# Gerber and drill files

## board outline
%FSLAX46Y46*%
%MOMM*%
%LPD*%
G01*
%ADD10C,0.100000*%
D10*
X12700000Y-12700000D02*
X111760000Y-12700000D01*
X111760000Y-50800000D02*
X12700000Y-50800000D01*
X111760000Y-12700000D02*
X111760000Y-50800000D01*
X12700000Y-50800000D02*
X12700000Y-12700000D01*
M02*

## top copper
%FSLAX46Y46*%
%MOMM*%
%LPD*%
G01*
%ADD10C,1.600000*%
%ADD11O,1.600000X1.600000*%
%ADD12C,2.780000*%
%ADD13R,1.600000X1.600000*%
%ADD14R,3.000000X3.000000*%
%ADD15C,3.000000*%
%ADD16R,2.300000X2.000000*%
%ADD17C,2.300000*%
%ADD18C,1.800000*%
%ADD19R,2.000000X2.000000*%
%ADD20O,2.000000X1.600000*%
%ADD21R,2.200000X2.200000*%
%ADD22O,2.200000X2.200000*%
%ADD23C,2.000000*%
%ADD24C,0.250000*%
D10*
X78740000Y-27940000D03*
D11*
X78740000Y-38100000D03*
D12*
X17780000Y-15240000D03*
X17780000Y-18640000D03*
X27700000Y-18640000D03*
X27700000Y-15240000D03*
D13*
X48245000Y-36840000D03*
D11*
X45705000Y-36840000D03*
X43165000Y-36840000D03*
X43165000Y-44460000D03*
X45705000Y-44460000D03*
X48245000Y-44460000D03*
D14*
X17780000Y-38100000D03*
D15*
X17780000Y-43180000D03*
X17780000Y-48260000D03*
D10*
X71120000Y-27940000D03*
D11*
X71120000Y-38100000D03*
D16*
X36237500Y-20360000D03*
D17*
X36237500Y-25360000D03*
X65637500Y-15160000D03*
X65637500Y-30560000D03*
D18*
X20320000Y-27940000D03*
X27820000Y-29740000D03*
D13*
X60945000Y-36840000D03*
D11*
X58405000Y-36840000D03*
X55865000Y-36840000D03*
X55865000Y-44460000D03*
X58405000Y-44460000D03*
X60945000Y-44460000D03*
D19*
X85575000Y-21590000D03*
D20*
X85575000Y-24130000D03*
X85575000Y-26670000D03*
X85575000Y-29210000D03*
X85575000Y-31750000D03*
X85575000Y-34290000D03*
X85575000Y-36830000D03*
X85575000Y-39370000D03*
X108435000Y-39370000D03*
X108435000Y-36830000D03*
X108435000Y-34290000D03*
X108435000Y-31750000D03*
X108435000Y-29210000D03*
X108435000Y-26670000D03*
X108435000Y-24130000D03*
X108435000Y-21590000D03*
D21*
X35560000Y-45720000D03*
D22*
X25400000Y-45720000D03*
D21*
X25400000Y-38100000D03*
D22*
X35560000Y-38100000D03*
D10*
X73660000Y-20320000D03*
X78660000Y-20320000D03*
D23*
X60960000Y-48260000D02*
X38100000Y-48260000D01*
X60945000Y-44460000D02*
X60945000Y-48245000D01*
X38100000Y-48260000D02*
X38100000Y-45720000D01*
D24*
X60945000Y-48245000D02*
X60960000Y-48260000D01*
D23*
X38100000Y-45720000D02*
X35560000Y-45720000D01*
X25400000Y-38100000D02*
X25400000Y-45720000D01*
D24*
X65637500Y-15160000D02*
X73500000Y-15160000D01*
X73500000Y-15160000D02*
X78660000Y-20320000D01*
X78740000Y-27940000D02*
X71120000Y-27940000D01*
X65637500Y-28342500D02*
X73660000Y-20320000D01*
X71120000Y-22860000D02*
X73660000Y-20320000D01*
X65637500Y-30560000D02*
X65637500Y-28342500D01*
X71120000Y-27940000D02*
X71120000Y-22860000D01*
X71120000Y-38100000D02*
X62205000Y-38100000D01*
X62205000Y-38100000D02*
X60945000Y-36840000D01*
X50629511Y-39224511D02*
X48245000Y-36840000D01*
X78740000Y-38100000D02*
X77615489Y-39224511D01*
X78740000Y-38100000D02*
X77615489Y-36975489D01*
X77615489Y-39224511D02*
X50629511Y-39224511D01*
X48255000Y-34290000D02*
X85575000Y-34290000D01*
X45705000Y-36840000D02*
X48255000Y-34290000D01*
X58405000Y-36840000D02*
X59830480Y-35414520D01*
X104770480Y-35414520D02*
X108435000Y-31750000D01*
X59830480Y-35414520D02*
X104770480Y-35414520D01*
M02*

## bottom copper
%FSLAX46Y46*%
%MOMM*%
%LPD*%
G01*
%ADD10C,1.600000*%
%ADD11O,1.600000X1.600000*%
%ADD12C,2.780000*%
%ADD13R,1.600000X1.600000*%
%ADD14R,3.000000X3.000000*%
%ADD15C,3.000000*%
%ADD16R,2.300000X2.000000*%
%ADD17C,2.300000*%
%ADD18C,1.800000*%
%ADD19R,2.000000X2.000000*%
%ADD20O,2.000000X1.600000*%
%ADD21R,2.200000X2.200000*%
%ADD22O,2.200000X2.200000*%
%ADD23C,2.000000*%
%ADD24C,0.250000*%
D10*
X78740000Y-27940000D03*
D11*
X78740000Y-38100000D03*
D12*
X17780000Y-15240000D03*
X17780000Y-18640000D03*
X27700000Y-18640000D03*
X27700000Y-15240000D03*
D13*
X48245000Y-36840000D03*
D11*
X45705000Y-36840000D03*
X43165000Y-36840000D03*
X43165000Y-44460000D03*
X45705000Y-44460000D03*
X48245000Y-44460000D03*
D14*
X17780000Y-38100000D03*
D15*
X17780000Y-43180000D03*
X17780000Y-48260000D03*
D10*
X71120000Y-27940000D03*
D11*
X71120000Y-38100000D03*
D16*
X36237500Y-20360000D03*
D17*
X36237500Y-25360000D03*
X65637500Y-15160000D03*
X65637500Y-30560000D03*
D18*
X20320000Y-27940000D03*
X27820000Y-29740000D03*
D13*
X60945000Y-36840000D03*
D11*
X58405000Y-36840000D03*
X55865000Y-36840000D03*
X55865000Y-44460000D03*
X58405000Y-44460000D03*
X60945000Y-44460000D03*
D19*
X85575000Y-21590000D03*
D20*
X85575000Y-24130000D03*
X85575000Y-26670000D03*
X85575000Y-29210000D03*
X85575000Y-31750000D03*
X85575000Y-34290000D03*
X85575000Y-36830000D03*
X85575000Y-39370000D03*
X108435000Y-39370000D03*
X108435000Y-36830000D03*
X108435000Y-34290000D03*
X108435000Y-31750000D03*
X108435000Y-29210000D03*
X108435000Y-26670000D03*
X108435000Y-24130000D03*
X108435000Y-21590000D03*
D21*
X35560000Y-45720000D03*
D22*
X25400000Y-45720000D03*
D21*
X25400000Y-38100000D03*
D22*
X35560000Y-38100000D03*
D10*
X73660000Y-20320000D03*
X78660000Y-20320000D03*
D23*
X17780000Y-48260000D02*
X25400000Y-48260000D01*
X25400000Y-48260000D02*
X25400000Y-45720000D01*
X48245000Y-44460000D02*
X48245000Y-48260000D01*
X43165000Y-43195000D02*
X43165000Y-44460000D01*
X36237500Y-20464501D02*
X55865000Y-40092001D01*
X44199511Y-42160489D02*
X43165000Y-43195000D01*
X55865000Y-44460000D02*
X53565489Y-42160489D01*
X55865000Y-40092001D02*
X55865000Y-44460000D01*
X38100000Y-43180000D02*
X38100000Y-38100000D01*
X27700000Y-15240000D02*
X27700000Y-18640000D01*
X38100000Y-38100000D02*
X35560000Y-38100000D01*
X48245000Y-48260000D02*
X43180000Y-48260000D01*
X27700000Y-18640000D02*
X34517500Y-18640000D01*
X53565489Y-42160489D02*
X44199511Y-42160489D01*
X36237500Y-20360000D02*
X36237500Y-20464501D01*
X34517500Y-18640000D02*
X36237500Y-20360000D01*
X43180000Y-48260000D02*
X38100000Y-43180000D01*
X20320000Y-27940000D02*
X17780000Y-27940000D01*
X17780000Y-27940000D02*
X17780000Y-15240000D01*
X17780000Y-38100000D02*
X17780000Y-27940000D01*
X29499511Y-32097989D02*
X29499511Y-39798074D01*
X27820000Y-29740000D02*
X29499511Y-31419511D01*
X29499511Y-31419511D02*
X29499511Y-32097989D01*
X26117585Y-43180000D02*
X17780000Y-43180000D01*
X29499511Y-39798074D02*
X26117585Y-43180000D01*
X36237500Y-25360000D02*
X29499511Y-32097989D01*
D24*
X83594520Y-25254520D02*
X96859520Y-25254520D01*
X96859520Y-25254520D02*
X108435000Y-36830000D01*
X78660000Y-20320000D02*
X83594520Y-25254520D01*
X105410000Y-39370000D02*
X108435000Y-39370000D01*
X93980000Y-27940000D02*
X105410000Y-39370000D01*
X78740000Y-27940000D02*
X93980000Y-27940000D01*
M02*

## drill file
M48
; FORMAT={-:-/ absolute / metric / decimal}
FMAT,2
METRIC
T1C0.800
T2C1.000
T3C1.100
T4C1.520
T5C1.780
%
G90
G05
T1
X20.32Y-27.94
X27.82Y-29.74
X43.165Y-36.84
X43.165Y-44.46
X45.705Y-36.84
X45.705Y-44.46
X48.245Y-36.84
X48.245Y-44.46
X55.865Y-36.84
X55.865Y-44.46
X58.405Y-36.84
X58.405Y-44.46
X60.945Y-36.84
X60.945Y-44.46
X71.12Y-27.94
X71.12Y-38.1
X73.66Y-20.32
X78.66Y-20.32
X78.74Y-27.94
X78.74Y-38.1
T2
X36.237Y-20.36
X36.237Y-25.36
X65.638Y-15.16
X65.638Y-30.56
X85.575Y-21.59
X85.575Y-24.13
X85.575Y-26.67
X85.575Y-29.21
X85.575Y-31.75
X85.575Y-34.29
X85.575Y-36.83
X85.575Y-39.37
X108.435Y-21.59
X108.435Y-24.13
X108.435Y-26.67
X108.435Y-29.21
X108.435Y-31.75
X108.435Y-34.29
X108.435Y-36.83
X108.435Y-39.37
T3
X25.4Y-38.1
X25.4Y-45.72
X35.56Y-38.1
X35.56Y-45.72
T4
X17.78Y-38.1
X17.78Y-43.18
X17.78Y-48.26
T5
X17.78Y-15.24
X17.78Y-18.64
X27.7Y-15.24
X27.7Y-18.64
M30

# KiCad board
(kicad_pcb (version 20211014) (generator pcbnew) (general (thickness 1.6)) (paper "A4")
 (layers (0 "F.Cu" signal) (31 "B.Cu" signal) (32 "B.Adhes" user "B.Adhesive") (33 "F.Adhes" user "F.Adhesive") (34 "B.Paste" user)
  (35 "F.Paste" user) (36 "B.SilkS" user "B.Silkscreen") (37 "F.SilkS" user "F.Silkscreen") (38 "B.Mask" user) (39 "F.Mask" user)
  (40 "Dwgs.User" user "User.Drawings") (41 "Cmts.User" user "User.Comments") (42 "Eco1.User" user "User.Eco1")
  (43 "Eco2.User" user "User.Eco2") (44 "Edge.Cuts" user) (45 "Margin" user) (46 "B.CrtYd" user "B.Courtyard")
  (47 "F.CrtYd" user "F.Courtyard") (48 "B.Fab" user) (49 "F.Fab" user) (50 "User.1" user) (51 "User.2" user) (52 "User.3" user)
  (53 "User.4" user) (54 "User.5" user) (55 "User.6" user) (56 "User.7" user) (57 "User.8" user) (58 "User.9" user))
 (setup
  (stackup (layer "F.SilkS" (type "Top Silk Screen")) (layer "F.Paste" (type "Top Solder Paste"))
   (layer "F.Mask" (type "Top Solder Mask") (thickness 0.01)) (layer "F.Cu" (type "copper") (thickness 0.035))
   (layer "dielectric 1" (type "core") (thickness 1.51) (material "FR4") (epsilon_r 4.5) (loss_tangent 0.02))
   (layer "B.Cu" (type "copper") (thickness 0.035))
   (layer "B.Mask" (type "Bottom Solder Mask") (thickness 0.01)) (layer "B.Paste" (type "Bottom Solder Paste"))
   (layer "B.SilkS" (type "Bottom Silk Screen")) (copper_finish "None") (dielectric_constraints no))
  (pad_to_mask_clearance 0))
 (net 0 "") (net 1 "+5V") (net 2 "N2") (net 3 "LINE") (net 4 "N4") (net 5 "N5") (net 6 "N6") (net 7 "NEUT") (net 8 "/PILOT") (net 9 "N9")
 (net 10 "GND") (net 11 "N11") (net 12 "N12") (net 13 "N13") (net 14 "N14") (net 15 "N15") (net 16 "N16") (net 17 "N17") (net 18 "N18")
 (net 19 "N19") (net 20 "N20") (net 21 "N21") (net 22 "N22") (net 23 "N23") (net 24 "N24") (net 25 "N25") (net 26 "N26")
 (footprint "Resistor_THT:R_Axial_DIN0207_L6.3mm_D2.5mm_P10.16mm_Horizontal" (layer "F.Cu") (at 78.74 27.94 -90)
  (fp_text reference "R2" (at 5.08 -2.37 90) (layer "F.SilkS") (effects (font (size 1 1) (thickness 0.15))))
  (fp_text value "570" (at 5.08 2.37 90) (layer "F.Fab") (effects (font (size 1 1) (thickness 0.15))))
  (pad "1" thru_hole circle (at 0 0 270) (size 1.6 1.6) (drill 0.8) (layers *.Cu *.Mask) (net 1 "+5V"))
  (pad "2" thru_hole oval (at 10.16 0 270) (size 1.6 1.6) (drill 0.8) (layers *.Cu *.Mask) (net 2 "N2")))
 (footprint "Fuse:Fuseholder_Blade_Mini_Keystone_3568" (layer "F.Cu") (at 17.78 15.24)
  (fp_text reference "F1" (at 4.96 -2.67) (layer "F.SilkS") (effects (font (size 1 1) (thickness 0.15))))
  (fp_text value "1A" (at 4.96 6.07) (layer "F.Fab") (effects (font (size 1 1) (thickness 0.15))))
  (pad "1" thru_hole circle (at 0 0) (size 2.78 2.78) (drill 1.78) (layers *.Cu *.Mask) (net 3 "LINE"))
  (pad "1" thru_hole circle (at 0 3.4) (size 2.78 2.78) (drill 1.78) (layers *.Cu *.Mask) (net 3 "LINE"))
  (pad "2" thru_hole circle (at 9.92 3.4) (size 2.78 2.78) (drill 1.78) (layers *.Cu *.Mask) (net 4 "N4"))
  (pad "2" thru_hole circle (at 9.92 0) (size 2.78 2.78) (drill 1.78) (layers *.Cu *.Mask) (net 4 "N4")))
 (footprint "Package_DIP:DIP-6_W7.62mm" (layer "F.Cu") (at 48.245 36.84 -90)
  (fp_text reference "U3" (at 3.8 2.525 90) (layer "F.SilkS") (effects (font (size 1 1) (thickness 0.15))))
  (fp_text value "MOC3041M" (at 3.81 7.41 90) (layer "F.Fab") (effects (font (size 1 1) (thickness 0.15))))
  (pad "1" thru_hole rect (at 0 0 270) (size 1.6 1.6) (drill 0.8) (layers *.Cu *.Mask) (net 2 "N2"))
  (pad "2" thru_hole oval (at 0 2.54 270) (size 1.6 1.6) (drill 0.8) (layers *.Cu *.Mask) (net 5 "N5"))
  (pad "3" thru_hole oval (at 0 5.08 270) (size 1.6 1.6) (drill 0.8) (layers *.Cu *.Mask) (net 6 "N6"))
  (pad "4" thru_hole oval (at 7.62 5.08 270) (size 1.6 1.6) (drill 0.8) (layers *.Cu *.Mask) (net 4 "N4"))
  (pad "5" thru_hole oval (at 7.62 2.54 270) (size 1.6 1.6) (drill 0.8) (layers *.Cu *.Mask) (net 4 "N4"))
  (pad "6" thru_hole oval (at 7.62 0 270) (size 1.6 1.6) (drill 0.8) (layers *.Cu *.Mask) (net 4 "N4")))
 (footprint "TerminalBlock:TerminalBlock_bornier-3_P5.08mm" (layer "F.Cu") (at 17.78 38.1 -90)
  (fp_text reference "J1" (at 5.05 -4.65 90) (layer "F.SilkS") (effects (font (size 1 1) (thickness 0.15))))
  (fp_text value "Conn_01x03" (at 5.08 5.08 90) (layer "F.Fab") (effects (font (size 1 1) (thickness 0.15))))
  (pad "1" thru_hole rect (at 0 0 270) (size 3 3) (drill 1.52) (layers *.Cu *.Mask) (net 3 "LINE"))
  (pad "2" thru_hole circle (at 5.08 0 270) (size 3 3) (drill 1.52) (layers *.Cu *.Mask) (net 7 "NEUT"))
  (pad "3" thru_hole circle (at 10.16 0 270) (size 3 3) (drill 1.52) (layers *.Cu *.Mask) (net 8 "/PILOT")))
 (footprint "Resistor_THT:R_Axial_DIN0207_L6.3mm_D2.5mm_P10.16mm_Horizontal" (layer "F.Cu") (at 71.12 27.94 -90)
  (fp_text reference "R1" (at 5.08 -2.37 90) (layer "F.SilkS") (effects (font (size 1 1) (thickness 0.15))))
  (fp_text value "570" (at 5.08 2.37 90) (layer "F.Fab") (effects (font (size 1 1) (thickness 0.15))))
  (pad "1" thru_hole circle (at 0 0 270) (size 1.6 1.6) (drill 0.8) (layers *.Cu *.Mask) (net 1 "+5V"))
  (pad "2" thru_hole oval (at 10.16 0 270) (size 1.6 1.6) (drill 0.8) (layers *.Cu *.Mask) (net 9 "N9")))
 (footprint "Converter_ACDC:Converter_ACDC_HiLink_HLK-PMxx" (layer "F.Cu") (at 36.2375 20.36)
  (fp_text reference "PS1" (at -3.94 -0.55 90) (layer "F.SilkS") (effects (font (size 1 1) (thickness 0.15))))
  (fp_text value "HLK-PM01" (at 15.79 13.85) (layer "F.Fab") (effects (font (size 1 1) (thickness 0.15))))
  (pad "1" thru_hole rect (at 0 0) (size 2.3 2) (drill 1) (layers *.Cu *.Mask) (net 4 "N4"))
  (pad "2" thru_hole circle (at 0 5) (size 2.3 2.3) (drill 1) (layers *.Cu *.Mask) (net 7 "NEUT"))
  (pad "3" thru_hole circle (at 29.4 -5.2) (size 2.3 2.3) (drill 1) (layers *.Cu *.Mask) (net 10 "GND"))
  (pad "4" thru_hole circle (at 29.4 10.2) (size 2.3 2.3) (drill 1) (layers *.Cu *.Mask) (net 1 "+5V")))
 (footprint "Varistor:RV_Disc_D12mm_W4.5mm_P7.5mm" (layer "F.Cu") (at 20.32 27.94)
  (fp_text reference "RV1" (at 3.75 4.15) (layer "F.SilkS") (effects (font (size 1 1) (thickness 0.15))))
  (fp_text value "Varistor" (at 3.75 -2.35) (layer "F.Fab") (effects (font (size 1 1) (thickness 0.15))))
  (pad "1" thru_hole circle (at 0 0) (size 1.8 1.8) (drill 0.8) (layers *.Cu *.Mask) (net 3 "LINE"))
  (pad "2" thru_hole circle (at 7.5 1.8) (size 1.8 1.8) (drill 0.8) (layers *.Cu *.Mask) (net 7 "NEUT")))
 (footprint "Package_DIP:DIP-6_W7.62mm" (layer "F.Cu") (at 60.945 36.84 -90)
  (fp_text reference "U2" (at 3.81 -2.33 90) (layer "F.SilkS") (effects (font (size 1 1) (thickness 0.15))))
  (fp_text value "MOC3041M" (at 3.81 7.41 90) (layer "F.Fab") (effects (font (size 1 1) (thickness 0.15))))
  (pad "1" thru_hole rect (at 0 0 270) (size 1.6 1.6) (drill 0.8) (layers *.Cu *.Mask) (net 9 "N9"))
  (pad "2" thru_hole oval (at 0 2.54 270) (size 1.6 1.6) (drill 0.8) (layers *.Cu *.Mask) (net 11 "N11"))
  (pad "3" thru_hole oval (at 0 5.08 270) (size 1.6 1.6) (drill 0.8) (layers *.Cu *.Mask) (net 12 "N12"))
  (pad "4" thru_hole oval (at 7.62 5.08 270) (size 1.6 1.6) (drill 0.8) (layers *.Cu *.Mask) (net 4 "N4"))
  (pad "5" thru_hole oval (at 7.62 2.54 270) (size 1.6 1.6) (drill 0.8) (layers *.Cu *.Mask) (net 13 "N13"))
  (pad "6" thru_hole oval (at 7.62 0 270) (size 1.6 1.6) (drill 0.8) (layers *.Cu *.Mask) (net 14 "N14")))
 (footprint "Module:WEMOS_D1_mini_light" (layer "F.Cu") (at 85.575 21.59)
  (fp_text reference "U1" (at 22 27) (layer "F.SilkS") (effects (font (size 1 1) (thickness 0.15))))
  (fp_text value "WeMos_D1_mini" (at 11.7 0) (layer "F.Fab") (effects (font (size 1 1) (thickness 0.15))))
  (pad "1" thru_hole rect (at 0 0) (size 2 2) (drill 1) (layers *.Cu *.Mask) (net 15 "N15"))
  (pad "2" thru_hole oval (at 0 2.54) (size 2 1.6) (drill 1) (layers *.Cu *.Mask) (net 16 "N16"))
  (pad "3" thru_hole oval (at 0 5.08) (size 2 1.6) (drill 1) (layers *.Cu *.Mask) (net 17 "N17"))
  (pad "4" thru_hole oval (at 0 7.62) (size 2 1.6) (drill 1) (layers *.Cu *.Mask) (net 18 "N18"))
  (pad "5" thru_hole oval (at 0 10.16) (size 2 1.6) (drill 1) (layers *.Cu *.Mask) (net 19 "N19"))
  (pad "6" thru_hole oval (at 0 12.7) (size 2 1.6) (drill 1) (layers *.Cu *.Mask) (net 5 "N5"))
  (pad "7" thru_hole oval (at 0 15.24) (size 2 1.6) (drill 1) (layers *.Cu *.Mask) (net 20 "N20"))
  (pad "8" thru_hole oval (at 0 17.78) (size 2 1.6) (drill 1) (layers *.Cu *.Mask) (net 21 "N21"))
  (pad "9" thru_hole oval (at 22.86 17.78) (size 2 1.6) (drill 1) (layers *.Cu *.Mask) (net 1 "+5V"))
  (pad "10" thru_hole oval (at 22.86 15.24) (size 2 1.6) (drill 1) (layers *.Cu *.Mask) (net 10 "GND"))
  (pad "11" thru_hole oval (at 22.86 12.7) (size 2 1.6) (drill 1) (layers *.Cu *.Mask) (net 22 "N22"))
  (pad "12" thru_hole oval (at 22.86 10.16) (size 2 1.6) (drill 1) (layers *.Cu *.Mask) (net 11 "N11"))
  (pad "13" thru_hole oval (at 22.86 7.62) (size 2 1.6) (drill 1) (layers *.Cu *.Mask) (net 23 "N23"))
  (pad "14" thru_hole oval (at 22.86 5.08) (size 2 1.6) (drill 1) (layers *.Cu *.Mask) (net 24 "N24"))
  (pad "15" thru_hole oval (at 22.86 2.54) (size 2 1.6) (drill 1) (layers *.Cu *.Mask) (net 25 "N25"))
  (pad "16" thru_hole oval (at 22.86 0) (size 2 1.6) (drill 1) (layers *.Cu *.Mask) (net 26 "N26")))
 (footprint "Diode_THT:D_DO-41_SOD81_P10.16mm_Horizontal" (layer "F.Cu") (at 35.56 45.72 180)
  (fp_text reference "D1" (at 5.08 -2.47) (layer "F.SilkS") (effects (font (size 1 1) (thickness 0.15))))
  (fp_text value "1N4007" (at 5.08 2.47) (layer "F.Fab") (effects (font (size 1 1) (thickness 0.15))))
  (pad "1" thru_hole rect (at 0 0 180) (size 2.2 2.2) (drill 1.1) (layers *.Cu *.Mask) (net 14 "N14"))
  (pad "2" thru_hole oval (at 10.16 0 180) (size 2.2 2.2) (drill 1.1) (layers *.Cu *.Mask) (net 8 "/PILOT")))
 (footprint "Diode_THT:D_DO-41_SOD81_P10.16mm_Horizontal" (layer "F.Cu") (at 25.4 38.1)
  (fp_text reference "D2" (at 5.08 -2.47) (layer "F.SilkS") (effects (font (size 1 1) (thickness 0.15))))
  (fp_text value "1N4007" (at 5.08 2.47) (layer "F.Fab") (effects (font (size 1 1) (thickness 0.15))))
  (pad "1" thru_hole rect (at 0 0) (size 2.2 2.2) (drill 1.1) (layers *.Cu *.Mask) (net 8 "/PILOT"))
  (pad "2" thru_hole oval (at 10.16 0) (size 2.2 2.2) (drill 1.1) (layers *.Cu *.Mask) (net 4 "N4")))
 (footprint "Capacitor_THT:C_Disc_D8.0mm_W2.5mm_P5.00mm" (layer "F.Cu") (at 73.66 20.32)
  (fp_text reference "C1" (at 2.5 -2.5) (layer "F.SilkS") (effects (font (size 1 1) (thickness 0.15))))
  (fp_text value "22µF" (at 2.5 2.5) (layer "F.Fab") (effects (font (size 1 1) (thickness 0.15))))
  (pad "1" thru_hole circle (at 0 0) (size 1.6 1.6) (drill 0.8) (layers *.Cu *.Mask) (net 1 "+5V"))
  (pad "2" thru_hole circle (at 5 0) (size 1.6 1.6) (drill 0.8) (layers *.Cu *.Mask) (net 10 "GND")))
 (gr_line (start 12.7 12.7) (end 111.76 12.7) (layer "Edge.Cuts") (width 0.1))
 (gr_line (start 111.76 50.8) (end 12.7 50.8) (layer "Edge.Cuts") (width 0.1))
 (gr_line (start 111.76 12.7) (end 111.76 50.8) (layer "Edge.Cuts") (width 0.1))
 (gr_line (start 12.7 50.8) (end 12.7 12.7) (layer "Edge.Cuts") (width 0.1))
 (segment (start 60.96 48.26) (end 38.1 48.26) (width 2) (layer "F.Cu") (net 14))
 (segment (start 60.945 44.46) (end 60.945 48.245) (width 2) (layer "F.Cu") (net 14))
 (segment (start 38.1 48.26) (end 38.1 45.72) (width 2) (layer "F.Cu") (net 14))
 (segment (start 60.945 48.245) (end 60.96 48.26) (width 0.25) (layer "F.Cu") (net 14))
 (segment (start 38.1 45.72) (end 35.56 45.72) (width 2) (layer "F.Cu") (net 14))
 (segment (start 25.4 38.1) (end 25.4 45.72) (width 2) (layer "F.Cu") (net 8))
 (segment (start 17.78 48.26) (end 25.4 48.26) (width 2) (layer "B.Cu") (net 8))
 (segment (start 25.4 48.26) (end 25.4 45.72) (width 2) (layer "B.Cu") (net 8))
 (segment (start 48.245 44.46) (end 48.245 48.26) (width 2) (layer "B.Cu") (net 4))
 (segment (start 43.165 43.195) (end 43.165 44.46) (width 2) (layer "B.Cu") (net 4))
 (segment (start 36.2375 20.464501) (end 55.865 40.092001) (width 2) (layer "B.Cu") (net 4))
 (segment (start 44.199511 42.160489) (end 43.165 43.195) (width 2) (layer "B.Cu") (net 4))
 (segment (start 55.865 44.46) (end 53.565489 42.160489) (width 2) (layer "B.Cu") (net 4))
 (segment (start 55.865 40.092001) (end 55.865 44.46) (width 2) (layer "B.Cu") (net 4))
 (segment (start 38.1 43.18) (end 38.1 38.1) (width 2) (layer "B.Cu") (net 4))
 (segment (start 27.7 15.24) (end 27.7 18.64) (width 2) (layer "B.Cu") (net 4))
 (segment (start 38.1 38.1) (end 35.56 38.1) (width 2) (layer "B.Cu") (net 4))
 (segment (start 48.245 48.26) (end 43.18 48.26) (width 2) (layer "B.Cu") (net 4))
 (segment (start 27.7 18.64) (end 34.5175 18.64) (width 2) (layer "B.Cu") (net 4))
 (segment (start 53.565489 42.160489) (end 44.199511 42.160489) (width 2) (layer "B.Cu") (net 4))
 (segment (start 36.2375 20.36) (end 36.2375 20.464501) (width 2) (layer "B.Cu") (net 4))
 (segment (start 34.5175 18.64) (end 36.2375 20.36) (width 2) (layer "B.Cu") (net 4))
 (segment (start 43.18 48.26) (end 38.1 43.18) (width 2) (layer "B.Cu") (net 4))
 (segment (start 20.32 27.94) (end 17.78 27.94) (width 2) (layer "B.Cu") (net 3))
 (segment (start 17.78 27.94) (end 17.78 15.24) (width 2) (layer "B.Cu") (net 3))
 (segment (start 17.78 38.1) (end 17.78 27.94) (width 2) (layer "B.Cu") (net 3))
 (segment (start 29.499511 32.097989) (end 29.499511 39.798074) (width 2) (layer "B.Cu") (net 7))
 (segment (start 27.82 29.74) (end 29.499511 31.419511) (width 2) (layer "B.Cu") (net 7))
 (segment (start 29.499511 31.419511) (end 29.499511 32.097989) (width 2) (layer "B.Cu") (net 7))
 (segment (start 26.117585 43.18) (end 17.78 43.18) (width 2) (layer "B.Cu") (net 7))
 (segment (start 29.499511 39.798074) (end 26.117585 43.18) (width 2) (layer "B.Cu") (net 7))
 (segment (start 36.2375 25.36) (end 29.499511 32.097989) (width 2) (layer "B.Cu") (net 7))
 (segment (start 65.6375 15.16) (end 73.5 15.16) (width 0.25) (layer "F.Cu") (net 10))
 (segment (start 73.5 15.16) (end 78.66 20.32) (width 0.25) (layer "F.Cu") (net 10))
 (segment (start 83.59452 25.25452) (end 96.85952 25.25452) (width 0.25) (layer "B.Cu") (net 10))
 (segment (start 96.85952 25.25452) (end 108.435 36.83) (width 0.25) (layer "B.Cu") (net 10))
 (segment (start 78.66 20.32) (end 83.59452 25.25452) (width 0.25) (layer "B.Cu") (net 10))
 (segment (start 78.74 27.94) (end 71.12 27.94) (width 0.25) (layer "F.Cu") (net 1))
 (segment (start 65.6375 28.3425) (end 73.66 20.32) (width 0.25) (layer "F.Cu") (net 1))
 (segment (start 71.12 22.86) (end 73.66 20.32) (width 0.25) (layer "F.Cu") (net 1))
 (segment (start 65.6375 30.56) (end 65.6375 28.3425) (width 0.25) (layer "F.Cu") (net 1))
 (segment (start 71.12 27.94) (end 71.12 22.86) (width 0.25) (layer "F.Cu") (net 1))
 (segment (start 105.41 39.37) (end 108.435 39.37) (width 0.25) (layer "B.Cu") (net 1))
 (segment (start 93.98 27.94) (end 105.41 39.37) (width 0.25) (layer "B.Cu") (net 1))
 (segment (start 78.74 27.94) (end 93.98 27.94) (width 0.25) (layer "B.Cu") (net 1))
 (segment (start 71.12 38.1) (end 62.205 38.1) (width 0.25) (layer "F.Cu") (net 9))
 (segment (start 62.205 38.1) (end 60.945 36.84) (width 0.25) (layer "F.Cu") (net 9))
 (segment (start 50.629511 39.224511) (end 48.245 36.84) (width 0.25) (layer "F.Cu") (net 2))
 (segment (start 78.74 38.1) (end 77.615489 39.224511) (width 0.25) (layer "F.Cu") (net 2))
 (segment (start 78.74 38.1) (end 77.615489 36.975489) (width 0.25) (layer "F.Cu") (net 2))
 (segment (start 77.615489 39.224511) (end 50.629511 39.224511) (width 0.25) (layer "F.Cu") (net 2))
 (segment (start 48.255 34.29) (end 85.575 34.29) (width 0.25) (layer "F.Cu") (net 5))
 (segment (start 45.705 36.84) (end 48.255 34.29) (width 0.25) (layer "F.Cu") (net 5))
 (segment (start 58.405 36.84) (end 59.83048 35.41452) (width 0.25) (layer "F.Cu") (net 11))
 (segment (start 104.77048 35.41452) (end 108.435 31.75) (width 0.25) (layer "F.Cu") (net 11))
 (segment (start 59.83048 35.41452) (end 104.77048 35.41452) (width 0.25) (layer "F.Cu") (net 11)))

